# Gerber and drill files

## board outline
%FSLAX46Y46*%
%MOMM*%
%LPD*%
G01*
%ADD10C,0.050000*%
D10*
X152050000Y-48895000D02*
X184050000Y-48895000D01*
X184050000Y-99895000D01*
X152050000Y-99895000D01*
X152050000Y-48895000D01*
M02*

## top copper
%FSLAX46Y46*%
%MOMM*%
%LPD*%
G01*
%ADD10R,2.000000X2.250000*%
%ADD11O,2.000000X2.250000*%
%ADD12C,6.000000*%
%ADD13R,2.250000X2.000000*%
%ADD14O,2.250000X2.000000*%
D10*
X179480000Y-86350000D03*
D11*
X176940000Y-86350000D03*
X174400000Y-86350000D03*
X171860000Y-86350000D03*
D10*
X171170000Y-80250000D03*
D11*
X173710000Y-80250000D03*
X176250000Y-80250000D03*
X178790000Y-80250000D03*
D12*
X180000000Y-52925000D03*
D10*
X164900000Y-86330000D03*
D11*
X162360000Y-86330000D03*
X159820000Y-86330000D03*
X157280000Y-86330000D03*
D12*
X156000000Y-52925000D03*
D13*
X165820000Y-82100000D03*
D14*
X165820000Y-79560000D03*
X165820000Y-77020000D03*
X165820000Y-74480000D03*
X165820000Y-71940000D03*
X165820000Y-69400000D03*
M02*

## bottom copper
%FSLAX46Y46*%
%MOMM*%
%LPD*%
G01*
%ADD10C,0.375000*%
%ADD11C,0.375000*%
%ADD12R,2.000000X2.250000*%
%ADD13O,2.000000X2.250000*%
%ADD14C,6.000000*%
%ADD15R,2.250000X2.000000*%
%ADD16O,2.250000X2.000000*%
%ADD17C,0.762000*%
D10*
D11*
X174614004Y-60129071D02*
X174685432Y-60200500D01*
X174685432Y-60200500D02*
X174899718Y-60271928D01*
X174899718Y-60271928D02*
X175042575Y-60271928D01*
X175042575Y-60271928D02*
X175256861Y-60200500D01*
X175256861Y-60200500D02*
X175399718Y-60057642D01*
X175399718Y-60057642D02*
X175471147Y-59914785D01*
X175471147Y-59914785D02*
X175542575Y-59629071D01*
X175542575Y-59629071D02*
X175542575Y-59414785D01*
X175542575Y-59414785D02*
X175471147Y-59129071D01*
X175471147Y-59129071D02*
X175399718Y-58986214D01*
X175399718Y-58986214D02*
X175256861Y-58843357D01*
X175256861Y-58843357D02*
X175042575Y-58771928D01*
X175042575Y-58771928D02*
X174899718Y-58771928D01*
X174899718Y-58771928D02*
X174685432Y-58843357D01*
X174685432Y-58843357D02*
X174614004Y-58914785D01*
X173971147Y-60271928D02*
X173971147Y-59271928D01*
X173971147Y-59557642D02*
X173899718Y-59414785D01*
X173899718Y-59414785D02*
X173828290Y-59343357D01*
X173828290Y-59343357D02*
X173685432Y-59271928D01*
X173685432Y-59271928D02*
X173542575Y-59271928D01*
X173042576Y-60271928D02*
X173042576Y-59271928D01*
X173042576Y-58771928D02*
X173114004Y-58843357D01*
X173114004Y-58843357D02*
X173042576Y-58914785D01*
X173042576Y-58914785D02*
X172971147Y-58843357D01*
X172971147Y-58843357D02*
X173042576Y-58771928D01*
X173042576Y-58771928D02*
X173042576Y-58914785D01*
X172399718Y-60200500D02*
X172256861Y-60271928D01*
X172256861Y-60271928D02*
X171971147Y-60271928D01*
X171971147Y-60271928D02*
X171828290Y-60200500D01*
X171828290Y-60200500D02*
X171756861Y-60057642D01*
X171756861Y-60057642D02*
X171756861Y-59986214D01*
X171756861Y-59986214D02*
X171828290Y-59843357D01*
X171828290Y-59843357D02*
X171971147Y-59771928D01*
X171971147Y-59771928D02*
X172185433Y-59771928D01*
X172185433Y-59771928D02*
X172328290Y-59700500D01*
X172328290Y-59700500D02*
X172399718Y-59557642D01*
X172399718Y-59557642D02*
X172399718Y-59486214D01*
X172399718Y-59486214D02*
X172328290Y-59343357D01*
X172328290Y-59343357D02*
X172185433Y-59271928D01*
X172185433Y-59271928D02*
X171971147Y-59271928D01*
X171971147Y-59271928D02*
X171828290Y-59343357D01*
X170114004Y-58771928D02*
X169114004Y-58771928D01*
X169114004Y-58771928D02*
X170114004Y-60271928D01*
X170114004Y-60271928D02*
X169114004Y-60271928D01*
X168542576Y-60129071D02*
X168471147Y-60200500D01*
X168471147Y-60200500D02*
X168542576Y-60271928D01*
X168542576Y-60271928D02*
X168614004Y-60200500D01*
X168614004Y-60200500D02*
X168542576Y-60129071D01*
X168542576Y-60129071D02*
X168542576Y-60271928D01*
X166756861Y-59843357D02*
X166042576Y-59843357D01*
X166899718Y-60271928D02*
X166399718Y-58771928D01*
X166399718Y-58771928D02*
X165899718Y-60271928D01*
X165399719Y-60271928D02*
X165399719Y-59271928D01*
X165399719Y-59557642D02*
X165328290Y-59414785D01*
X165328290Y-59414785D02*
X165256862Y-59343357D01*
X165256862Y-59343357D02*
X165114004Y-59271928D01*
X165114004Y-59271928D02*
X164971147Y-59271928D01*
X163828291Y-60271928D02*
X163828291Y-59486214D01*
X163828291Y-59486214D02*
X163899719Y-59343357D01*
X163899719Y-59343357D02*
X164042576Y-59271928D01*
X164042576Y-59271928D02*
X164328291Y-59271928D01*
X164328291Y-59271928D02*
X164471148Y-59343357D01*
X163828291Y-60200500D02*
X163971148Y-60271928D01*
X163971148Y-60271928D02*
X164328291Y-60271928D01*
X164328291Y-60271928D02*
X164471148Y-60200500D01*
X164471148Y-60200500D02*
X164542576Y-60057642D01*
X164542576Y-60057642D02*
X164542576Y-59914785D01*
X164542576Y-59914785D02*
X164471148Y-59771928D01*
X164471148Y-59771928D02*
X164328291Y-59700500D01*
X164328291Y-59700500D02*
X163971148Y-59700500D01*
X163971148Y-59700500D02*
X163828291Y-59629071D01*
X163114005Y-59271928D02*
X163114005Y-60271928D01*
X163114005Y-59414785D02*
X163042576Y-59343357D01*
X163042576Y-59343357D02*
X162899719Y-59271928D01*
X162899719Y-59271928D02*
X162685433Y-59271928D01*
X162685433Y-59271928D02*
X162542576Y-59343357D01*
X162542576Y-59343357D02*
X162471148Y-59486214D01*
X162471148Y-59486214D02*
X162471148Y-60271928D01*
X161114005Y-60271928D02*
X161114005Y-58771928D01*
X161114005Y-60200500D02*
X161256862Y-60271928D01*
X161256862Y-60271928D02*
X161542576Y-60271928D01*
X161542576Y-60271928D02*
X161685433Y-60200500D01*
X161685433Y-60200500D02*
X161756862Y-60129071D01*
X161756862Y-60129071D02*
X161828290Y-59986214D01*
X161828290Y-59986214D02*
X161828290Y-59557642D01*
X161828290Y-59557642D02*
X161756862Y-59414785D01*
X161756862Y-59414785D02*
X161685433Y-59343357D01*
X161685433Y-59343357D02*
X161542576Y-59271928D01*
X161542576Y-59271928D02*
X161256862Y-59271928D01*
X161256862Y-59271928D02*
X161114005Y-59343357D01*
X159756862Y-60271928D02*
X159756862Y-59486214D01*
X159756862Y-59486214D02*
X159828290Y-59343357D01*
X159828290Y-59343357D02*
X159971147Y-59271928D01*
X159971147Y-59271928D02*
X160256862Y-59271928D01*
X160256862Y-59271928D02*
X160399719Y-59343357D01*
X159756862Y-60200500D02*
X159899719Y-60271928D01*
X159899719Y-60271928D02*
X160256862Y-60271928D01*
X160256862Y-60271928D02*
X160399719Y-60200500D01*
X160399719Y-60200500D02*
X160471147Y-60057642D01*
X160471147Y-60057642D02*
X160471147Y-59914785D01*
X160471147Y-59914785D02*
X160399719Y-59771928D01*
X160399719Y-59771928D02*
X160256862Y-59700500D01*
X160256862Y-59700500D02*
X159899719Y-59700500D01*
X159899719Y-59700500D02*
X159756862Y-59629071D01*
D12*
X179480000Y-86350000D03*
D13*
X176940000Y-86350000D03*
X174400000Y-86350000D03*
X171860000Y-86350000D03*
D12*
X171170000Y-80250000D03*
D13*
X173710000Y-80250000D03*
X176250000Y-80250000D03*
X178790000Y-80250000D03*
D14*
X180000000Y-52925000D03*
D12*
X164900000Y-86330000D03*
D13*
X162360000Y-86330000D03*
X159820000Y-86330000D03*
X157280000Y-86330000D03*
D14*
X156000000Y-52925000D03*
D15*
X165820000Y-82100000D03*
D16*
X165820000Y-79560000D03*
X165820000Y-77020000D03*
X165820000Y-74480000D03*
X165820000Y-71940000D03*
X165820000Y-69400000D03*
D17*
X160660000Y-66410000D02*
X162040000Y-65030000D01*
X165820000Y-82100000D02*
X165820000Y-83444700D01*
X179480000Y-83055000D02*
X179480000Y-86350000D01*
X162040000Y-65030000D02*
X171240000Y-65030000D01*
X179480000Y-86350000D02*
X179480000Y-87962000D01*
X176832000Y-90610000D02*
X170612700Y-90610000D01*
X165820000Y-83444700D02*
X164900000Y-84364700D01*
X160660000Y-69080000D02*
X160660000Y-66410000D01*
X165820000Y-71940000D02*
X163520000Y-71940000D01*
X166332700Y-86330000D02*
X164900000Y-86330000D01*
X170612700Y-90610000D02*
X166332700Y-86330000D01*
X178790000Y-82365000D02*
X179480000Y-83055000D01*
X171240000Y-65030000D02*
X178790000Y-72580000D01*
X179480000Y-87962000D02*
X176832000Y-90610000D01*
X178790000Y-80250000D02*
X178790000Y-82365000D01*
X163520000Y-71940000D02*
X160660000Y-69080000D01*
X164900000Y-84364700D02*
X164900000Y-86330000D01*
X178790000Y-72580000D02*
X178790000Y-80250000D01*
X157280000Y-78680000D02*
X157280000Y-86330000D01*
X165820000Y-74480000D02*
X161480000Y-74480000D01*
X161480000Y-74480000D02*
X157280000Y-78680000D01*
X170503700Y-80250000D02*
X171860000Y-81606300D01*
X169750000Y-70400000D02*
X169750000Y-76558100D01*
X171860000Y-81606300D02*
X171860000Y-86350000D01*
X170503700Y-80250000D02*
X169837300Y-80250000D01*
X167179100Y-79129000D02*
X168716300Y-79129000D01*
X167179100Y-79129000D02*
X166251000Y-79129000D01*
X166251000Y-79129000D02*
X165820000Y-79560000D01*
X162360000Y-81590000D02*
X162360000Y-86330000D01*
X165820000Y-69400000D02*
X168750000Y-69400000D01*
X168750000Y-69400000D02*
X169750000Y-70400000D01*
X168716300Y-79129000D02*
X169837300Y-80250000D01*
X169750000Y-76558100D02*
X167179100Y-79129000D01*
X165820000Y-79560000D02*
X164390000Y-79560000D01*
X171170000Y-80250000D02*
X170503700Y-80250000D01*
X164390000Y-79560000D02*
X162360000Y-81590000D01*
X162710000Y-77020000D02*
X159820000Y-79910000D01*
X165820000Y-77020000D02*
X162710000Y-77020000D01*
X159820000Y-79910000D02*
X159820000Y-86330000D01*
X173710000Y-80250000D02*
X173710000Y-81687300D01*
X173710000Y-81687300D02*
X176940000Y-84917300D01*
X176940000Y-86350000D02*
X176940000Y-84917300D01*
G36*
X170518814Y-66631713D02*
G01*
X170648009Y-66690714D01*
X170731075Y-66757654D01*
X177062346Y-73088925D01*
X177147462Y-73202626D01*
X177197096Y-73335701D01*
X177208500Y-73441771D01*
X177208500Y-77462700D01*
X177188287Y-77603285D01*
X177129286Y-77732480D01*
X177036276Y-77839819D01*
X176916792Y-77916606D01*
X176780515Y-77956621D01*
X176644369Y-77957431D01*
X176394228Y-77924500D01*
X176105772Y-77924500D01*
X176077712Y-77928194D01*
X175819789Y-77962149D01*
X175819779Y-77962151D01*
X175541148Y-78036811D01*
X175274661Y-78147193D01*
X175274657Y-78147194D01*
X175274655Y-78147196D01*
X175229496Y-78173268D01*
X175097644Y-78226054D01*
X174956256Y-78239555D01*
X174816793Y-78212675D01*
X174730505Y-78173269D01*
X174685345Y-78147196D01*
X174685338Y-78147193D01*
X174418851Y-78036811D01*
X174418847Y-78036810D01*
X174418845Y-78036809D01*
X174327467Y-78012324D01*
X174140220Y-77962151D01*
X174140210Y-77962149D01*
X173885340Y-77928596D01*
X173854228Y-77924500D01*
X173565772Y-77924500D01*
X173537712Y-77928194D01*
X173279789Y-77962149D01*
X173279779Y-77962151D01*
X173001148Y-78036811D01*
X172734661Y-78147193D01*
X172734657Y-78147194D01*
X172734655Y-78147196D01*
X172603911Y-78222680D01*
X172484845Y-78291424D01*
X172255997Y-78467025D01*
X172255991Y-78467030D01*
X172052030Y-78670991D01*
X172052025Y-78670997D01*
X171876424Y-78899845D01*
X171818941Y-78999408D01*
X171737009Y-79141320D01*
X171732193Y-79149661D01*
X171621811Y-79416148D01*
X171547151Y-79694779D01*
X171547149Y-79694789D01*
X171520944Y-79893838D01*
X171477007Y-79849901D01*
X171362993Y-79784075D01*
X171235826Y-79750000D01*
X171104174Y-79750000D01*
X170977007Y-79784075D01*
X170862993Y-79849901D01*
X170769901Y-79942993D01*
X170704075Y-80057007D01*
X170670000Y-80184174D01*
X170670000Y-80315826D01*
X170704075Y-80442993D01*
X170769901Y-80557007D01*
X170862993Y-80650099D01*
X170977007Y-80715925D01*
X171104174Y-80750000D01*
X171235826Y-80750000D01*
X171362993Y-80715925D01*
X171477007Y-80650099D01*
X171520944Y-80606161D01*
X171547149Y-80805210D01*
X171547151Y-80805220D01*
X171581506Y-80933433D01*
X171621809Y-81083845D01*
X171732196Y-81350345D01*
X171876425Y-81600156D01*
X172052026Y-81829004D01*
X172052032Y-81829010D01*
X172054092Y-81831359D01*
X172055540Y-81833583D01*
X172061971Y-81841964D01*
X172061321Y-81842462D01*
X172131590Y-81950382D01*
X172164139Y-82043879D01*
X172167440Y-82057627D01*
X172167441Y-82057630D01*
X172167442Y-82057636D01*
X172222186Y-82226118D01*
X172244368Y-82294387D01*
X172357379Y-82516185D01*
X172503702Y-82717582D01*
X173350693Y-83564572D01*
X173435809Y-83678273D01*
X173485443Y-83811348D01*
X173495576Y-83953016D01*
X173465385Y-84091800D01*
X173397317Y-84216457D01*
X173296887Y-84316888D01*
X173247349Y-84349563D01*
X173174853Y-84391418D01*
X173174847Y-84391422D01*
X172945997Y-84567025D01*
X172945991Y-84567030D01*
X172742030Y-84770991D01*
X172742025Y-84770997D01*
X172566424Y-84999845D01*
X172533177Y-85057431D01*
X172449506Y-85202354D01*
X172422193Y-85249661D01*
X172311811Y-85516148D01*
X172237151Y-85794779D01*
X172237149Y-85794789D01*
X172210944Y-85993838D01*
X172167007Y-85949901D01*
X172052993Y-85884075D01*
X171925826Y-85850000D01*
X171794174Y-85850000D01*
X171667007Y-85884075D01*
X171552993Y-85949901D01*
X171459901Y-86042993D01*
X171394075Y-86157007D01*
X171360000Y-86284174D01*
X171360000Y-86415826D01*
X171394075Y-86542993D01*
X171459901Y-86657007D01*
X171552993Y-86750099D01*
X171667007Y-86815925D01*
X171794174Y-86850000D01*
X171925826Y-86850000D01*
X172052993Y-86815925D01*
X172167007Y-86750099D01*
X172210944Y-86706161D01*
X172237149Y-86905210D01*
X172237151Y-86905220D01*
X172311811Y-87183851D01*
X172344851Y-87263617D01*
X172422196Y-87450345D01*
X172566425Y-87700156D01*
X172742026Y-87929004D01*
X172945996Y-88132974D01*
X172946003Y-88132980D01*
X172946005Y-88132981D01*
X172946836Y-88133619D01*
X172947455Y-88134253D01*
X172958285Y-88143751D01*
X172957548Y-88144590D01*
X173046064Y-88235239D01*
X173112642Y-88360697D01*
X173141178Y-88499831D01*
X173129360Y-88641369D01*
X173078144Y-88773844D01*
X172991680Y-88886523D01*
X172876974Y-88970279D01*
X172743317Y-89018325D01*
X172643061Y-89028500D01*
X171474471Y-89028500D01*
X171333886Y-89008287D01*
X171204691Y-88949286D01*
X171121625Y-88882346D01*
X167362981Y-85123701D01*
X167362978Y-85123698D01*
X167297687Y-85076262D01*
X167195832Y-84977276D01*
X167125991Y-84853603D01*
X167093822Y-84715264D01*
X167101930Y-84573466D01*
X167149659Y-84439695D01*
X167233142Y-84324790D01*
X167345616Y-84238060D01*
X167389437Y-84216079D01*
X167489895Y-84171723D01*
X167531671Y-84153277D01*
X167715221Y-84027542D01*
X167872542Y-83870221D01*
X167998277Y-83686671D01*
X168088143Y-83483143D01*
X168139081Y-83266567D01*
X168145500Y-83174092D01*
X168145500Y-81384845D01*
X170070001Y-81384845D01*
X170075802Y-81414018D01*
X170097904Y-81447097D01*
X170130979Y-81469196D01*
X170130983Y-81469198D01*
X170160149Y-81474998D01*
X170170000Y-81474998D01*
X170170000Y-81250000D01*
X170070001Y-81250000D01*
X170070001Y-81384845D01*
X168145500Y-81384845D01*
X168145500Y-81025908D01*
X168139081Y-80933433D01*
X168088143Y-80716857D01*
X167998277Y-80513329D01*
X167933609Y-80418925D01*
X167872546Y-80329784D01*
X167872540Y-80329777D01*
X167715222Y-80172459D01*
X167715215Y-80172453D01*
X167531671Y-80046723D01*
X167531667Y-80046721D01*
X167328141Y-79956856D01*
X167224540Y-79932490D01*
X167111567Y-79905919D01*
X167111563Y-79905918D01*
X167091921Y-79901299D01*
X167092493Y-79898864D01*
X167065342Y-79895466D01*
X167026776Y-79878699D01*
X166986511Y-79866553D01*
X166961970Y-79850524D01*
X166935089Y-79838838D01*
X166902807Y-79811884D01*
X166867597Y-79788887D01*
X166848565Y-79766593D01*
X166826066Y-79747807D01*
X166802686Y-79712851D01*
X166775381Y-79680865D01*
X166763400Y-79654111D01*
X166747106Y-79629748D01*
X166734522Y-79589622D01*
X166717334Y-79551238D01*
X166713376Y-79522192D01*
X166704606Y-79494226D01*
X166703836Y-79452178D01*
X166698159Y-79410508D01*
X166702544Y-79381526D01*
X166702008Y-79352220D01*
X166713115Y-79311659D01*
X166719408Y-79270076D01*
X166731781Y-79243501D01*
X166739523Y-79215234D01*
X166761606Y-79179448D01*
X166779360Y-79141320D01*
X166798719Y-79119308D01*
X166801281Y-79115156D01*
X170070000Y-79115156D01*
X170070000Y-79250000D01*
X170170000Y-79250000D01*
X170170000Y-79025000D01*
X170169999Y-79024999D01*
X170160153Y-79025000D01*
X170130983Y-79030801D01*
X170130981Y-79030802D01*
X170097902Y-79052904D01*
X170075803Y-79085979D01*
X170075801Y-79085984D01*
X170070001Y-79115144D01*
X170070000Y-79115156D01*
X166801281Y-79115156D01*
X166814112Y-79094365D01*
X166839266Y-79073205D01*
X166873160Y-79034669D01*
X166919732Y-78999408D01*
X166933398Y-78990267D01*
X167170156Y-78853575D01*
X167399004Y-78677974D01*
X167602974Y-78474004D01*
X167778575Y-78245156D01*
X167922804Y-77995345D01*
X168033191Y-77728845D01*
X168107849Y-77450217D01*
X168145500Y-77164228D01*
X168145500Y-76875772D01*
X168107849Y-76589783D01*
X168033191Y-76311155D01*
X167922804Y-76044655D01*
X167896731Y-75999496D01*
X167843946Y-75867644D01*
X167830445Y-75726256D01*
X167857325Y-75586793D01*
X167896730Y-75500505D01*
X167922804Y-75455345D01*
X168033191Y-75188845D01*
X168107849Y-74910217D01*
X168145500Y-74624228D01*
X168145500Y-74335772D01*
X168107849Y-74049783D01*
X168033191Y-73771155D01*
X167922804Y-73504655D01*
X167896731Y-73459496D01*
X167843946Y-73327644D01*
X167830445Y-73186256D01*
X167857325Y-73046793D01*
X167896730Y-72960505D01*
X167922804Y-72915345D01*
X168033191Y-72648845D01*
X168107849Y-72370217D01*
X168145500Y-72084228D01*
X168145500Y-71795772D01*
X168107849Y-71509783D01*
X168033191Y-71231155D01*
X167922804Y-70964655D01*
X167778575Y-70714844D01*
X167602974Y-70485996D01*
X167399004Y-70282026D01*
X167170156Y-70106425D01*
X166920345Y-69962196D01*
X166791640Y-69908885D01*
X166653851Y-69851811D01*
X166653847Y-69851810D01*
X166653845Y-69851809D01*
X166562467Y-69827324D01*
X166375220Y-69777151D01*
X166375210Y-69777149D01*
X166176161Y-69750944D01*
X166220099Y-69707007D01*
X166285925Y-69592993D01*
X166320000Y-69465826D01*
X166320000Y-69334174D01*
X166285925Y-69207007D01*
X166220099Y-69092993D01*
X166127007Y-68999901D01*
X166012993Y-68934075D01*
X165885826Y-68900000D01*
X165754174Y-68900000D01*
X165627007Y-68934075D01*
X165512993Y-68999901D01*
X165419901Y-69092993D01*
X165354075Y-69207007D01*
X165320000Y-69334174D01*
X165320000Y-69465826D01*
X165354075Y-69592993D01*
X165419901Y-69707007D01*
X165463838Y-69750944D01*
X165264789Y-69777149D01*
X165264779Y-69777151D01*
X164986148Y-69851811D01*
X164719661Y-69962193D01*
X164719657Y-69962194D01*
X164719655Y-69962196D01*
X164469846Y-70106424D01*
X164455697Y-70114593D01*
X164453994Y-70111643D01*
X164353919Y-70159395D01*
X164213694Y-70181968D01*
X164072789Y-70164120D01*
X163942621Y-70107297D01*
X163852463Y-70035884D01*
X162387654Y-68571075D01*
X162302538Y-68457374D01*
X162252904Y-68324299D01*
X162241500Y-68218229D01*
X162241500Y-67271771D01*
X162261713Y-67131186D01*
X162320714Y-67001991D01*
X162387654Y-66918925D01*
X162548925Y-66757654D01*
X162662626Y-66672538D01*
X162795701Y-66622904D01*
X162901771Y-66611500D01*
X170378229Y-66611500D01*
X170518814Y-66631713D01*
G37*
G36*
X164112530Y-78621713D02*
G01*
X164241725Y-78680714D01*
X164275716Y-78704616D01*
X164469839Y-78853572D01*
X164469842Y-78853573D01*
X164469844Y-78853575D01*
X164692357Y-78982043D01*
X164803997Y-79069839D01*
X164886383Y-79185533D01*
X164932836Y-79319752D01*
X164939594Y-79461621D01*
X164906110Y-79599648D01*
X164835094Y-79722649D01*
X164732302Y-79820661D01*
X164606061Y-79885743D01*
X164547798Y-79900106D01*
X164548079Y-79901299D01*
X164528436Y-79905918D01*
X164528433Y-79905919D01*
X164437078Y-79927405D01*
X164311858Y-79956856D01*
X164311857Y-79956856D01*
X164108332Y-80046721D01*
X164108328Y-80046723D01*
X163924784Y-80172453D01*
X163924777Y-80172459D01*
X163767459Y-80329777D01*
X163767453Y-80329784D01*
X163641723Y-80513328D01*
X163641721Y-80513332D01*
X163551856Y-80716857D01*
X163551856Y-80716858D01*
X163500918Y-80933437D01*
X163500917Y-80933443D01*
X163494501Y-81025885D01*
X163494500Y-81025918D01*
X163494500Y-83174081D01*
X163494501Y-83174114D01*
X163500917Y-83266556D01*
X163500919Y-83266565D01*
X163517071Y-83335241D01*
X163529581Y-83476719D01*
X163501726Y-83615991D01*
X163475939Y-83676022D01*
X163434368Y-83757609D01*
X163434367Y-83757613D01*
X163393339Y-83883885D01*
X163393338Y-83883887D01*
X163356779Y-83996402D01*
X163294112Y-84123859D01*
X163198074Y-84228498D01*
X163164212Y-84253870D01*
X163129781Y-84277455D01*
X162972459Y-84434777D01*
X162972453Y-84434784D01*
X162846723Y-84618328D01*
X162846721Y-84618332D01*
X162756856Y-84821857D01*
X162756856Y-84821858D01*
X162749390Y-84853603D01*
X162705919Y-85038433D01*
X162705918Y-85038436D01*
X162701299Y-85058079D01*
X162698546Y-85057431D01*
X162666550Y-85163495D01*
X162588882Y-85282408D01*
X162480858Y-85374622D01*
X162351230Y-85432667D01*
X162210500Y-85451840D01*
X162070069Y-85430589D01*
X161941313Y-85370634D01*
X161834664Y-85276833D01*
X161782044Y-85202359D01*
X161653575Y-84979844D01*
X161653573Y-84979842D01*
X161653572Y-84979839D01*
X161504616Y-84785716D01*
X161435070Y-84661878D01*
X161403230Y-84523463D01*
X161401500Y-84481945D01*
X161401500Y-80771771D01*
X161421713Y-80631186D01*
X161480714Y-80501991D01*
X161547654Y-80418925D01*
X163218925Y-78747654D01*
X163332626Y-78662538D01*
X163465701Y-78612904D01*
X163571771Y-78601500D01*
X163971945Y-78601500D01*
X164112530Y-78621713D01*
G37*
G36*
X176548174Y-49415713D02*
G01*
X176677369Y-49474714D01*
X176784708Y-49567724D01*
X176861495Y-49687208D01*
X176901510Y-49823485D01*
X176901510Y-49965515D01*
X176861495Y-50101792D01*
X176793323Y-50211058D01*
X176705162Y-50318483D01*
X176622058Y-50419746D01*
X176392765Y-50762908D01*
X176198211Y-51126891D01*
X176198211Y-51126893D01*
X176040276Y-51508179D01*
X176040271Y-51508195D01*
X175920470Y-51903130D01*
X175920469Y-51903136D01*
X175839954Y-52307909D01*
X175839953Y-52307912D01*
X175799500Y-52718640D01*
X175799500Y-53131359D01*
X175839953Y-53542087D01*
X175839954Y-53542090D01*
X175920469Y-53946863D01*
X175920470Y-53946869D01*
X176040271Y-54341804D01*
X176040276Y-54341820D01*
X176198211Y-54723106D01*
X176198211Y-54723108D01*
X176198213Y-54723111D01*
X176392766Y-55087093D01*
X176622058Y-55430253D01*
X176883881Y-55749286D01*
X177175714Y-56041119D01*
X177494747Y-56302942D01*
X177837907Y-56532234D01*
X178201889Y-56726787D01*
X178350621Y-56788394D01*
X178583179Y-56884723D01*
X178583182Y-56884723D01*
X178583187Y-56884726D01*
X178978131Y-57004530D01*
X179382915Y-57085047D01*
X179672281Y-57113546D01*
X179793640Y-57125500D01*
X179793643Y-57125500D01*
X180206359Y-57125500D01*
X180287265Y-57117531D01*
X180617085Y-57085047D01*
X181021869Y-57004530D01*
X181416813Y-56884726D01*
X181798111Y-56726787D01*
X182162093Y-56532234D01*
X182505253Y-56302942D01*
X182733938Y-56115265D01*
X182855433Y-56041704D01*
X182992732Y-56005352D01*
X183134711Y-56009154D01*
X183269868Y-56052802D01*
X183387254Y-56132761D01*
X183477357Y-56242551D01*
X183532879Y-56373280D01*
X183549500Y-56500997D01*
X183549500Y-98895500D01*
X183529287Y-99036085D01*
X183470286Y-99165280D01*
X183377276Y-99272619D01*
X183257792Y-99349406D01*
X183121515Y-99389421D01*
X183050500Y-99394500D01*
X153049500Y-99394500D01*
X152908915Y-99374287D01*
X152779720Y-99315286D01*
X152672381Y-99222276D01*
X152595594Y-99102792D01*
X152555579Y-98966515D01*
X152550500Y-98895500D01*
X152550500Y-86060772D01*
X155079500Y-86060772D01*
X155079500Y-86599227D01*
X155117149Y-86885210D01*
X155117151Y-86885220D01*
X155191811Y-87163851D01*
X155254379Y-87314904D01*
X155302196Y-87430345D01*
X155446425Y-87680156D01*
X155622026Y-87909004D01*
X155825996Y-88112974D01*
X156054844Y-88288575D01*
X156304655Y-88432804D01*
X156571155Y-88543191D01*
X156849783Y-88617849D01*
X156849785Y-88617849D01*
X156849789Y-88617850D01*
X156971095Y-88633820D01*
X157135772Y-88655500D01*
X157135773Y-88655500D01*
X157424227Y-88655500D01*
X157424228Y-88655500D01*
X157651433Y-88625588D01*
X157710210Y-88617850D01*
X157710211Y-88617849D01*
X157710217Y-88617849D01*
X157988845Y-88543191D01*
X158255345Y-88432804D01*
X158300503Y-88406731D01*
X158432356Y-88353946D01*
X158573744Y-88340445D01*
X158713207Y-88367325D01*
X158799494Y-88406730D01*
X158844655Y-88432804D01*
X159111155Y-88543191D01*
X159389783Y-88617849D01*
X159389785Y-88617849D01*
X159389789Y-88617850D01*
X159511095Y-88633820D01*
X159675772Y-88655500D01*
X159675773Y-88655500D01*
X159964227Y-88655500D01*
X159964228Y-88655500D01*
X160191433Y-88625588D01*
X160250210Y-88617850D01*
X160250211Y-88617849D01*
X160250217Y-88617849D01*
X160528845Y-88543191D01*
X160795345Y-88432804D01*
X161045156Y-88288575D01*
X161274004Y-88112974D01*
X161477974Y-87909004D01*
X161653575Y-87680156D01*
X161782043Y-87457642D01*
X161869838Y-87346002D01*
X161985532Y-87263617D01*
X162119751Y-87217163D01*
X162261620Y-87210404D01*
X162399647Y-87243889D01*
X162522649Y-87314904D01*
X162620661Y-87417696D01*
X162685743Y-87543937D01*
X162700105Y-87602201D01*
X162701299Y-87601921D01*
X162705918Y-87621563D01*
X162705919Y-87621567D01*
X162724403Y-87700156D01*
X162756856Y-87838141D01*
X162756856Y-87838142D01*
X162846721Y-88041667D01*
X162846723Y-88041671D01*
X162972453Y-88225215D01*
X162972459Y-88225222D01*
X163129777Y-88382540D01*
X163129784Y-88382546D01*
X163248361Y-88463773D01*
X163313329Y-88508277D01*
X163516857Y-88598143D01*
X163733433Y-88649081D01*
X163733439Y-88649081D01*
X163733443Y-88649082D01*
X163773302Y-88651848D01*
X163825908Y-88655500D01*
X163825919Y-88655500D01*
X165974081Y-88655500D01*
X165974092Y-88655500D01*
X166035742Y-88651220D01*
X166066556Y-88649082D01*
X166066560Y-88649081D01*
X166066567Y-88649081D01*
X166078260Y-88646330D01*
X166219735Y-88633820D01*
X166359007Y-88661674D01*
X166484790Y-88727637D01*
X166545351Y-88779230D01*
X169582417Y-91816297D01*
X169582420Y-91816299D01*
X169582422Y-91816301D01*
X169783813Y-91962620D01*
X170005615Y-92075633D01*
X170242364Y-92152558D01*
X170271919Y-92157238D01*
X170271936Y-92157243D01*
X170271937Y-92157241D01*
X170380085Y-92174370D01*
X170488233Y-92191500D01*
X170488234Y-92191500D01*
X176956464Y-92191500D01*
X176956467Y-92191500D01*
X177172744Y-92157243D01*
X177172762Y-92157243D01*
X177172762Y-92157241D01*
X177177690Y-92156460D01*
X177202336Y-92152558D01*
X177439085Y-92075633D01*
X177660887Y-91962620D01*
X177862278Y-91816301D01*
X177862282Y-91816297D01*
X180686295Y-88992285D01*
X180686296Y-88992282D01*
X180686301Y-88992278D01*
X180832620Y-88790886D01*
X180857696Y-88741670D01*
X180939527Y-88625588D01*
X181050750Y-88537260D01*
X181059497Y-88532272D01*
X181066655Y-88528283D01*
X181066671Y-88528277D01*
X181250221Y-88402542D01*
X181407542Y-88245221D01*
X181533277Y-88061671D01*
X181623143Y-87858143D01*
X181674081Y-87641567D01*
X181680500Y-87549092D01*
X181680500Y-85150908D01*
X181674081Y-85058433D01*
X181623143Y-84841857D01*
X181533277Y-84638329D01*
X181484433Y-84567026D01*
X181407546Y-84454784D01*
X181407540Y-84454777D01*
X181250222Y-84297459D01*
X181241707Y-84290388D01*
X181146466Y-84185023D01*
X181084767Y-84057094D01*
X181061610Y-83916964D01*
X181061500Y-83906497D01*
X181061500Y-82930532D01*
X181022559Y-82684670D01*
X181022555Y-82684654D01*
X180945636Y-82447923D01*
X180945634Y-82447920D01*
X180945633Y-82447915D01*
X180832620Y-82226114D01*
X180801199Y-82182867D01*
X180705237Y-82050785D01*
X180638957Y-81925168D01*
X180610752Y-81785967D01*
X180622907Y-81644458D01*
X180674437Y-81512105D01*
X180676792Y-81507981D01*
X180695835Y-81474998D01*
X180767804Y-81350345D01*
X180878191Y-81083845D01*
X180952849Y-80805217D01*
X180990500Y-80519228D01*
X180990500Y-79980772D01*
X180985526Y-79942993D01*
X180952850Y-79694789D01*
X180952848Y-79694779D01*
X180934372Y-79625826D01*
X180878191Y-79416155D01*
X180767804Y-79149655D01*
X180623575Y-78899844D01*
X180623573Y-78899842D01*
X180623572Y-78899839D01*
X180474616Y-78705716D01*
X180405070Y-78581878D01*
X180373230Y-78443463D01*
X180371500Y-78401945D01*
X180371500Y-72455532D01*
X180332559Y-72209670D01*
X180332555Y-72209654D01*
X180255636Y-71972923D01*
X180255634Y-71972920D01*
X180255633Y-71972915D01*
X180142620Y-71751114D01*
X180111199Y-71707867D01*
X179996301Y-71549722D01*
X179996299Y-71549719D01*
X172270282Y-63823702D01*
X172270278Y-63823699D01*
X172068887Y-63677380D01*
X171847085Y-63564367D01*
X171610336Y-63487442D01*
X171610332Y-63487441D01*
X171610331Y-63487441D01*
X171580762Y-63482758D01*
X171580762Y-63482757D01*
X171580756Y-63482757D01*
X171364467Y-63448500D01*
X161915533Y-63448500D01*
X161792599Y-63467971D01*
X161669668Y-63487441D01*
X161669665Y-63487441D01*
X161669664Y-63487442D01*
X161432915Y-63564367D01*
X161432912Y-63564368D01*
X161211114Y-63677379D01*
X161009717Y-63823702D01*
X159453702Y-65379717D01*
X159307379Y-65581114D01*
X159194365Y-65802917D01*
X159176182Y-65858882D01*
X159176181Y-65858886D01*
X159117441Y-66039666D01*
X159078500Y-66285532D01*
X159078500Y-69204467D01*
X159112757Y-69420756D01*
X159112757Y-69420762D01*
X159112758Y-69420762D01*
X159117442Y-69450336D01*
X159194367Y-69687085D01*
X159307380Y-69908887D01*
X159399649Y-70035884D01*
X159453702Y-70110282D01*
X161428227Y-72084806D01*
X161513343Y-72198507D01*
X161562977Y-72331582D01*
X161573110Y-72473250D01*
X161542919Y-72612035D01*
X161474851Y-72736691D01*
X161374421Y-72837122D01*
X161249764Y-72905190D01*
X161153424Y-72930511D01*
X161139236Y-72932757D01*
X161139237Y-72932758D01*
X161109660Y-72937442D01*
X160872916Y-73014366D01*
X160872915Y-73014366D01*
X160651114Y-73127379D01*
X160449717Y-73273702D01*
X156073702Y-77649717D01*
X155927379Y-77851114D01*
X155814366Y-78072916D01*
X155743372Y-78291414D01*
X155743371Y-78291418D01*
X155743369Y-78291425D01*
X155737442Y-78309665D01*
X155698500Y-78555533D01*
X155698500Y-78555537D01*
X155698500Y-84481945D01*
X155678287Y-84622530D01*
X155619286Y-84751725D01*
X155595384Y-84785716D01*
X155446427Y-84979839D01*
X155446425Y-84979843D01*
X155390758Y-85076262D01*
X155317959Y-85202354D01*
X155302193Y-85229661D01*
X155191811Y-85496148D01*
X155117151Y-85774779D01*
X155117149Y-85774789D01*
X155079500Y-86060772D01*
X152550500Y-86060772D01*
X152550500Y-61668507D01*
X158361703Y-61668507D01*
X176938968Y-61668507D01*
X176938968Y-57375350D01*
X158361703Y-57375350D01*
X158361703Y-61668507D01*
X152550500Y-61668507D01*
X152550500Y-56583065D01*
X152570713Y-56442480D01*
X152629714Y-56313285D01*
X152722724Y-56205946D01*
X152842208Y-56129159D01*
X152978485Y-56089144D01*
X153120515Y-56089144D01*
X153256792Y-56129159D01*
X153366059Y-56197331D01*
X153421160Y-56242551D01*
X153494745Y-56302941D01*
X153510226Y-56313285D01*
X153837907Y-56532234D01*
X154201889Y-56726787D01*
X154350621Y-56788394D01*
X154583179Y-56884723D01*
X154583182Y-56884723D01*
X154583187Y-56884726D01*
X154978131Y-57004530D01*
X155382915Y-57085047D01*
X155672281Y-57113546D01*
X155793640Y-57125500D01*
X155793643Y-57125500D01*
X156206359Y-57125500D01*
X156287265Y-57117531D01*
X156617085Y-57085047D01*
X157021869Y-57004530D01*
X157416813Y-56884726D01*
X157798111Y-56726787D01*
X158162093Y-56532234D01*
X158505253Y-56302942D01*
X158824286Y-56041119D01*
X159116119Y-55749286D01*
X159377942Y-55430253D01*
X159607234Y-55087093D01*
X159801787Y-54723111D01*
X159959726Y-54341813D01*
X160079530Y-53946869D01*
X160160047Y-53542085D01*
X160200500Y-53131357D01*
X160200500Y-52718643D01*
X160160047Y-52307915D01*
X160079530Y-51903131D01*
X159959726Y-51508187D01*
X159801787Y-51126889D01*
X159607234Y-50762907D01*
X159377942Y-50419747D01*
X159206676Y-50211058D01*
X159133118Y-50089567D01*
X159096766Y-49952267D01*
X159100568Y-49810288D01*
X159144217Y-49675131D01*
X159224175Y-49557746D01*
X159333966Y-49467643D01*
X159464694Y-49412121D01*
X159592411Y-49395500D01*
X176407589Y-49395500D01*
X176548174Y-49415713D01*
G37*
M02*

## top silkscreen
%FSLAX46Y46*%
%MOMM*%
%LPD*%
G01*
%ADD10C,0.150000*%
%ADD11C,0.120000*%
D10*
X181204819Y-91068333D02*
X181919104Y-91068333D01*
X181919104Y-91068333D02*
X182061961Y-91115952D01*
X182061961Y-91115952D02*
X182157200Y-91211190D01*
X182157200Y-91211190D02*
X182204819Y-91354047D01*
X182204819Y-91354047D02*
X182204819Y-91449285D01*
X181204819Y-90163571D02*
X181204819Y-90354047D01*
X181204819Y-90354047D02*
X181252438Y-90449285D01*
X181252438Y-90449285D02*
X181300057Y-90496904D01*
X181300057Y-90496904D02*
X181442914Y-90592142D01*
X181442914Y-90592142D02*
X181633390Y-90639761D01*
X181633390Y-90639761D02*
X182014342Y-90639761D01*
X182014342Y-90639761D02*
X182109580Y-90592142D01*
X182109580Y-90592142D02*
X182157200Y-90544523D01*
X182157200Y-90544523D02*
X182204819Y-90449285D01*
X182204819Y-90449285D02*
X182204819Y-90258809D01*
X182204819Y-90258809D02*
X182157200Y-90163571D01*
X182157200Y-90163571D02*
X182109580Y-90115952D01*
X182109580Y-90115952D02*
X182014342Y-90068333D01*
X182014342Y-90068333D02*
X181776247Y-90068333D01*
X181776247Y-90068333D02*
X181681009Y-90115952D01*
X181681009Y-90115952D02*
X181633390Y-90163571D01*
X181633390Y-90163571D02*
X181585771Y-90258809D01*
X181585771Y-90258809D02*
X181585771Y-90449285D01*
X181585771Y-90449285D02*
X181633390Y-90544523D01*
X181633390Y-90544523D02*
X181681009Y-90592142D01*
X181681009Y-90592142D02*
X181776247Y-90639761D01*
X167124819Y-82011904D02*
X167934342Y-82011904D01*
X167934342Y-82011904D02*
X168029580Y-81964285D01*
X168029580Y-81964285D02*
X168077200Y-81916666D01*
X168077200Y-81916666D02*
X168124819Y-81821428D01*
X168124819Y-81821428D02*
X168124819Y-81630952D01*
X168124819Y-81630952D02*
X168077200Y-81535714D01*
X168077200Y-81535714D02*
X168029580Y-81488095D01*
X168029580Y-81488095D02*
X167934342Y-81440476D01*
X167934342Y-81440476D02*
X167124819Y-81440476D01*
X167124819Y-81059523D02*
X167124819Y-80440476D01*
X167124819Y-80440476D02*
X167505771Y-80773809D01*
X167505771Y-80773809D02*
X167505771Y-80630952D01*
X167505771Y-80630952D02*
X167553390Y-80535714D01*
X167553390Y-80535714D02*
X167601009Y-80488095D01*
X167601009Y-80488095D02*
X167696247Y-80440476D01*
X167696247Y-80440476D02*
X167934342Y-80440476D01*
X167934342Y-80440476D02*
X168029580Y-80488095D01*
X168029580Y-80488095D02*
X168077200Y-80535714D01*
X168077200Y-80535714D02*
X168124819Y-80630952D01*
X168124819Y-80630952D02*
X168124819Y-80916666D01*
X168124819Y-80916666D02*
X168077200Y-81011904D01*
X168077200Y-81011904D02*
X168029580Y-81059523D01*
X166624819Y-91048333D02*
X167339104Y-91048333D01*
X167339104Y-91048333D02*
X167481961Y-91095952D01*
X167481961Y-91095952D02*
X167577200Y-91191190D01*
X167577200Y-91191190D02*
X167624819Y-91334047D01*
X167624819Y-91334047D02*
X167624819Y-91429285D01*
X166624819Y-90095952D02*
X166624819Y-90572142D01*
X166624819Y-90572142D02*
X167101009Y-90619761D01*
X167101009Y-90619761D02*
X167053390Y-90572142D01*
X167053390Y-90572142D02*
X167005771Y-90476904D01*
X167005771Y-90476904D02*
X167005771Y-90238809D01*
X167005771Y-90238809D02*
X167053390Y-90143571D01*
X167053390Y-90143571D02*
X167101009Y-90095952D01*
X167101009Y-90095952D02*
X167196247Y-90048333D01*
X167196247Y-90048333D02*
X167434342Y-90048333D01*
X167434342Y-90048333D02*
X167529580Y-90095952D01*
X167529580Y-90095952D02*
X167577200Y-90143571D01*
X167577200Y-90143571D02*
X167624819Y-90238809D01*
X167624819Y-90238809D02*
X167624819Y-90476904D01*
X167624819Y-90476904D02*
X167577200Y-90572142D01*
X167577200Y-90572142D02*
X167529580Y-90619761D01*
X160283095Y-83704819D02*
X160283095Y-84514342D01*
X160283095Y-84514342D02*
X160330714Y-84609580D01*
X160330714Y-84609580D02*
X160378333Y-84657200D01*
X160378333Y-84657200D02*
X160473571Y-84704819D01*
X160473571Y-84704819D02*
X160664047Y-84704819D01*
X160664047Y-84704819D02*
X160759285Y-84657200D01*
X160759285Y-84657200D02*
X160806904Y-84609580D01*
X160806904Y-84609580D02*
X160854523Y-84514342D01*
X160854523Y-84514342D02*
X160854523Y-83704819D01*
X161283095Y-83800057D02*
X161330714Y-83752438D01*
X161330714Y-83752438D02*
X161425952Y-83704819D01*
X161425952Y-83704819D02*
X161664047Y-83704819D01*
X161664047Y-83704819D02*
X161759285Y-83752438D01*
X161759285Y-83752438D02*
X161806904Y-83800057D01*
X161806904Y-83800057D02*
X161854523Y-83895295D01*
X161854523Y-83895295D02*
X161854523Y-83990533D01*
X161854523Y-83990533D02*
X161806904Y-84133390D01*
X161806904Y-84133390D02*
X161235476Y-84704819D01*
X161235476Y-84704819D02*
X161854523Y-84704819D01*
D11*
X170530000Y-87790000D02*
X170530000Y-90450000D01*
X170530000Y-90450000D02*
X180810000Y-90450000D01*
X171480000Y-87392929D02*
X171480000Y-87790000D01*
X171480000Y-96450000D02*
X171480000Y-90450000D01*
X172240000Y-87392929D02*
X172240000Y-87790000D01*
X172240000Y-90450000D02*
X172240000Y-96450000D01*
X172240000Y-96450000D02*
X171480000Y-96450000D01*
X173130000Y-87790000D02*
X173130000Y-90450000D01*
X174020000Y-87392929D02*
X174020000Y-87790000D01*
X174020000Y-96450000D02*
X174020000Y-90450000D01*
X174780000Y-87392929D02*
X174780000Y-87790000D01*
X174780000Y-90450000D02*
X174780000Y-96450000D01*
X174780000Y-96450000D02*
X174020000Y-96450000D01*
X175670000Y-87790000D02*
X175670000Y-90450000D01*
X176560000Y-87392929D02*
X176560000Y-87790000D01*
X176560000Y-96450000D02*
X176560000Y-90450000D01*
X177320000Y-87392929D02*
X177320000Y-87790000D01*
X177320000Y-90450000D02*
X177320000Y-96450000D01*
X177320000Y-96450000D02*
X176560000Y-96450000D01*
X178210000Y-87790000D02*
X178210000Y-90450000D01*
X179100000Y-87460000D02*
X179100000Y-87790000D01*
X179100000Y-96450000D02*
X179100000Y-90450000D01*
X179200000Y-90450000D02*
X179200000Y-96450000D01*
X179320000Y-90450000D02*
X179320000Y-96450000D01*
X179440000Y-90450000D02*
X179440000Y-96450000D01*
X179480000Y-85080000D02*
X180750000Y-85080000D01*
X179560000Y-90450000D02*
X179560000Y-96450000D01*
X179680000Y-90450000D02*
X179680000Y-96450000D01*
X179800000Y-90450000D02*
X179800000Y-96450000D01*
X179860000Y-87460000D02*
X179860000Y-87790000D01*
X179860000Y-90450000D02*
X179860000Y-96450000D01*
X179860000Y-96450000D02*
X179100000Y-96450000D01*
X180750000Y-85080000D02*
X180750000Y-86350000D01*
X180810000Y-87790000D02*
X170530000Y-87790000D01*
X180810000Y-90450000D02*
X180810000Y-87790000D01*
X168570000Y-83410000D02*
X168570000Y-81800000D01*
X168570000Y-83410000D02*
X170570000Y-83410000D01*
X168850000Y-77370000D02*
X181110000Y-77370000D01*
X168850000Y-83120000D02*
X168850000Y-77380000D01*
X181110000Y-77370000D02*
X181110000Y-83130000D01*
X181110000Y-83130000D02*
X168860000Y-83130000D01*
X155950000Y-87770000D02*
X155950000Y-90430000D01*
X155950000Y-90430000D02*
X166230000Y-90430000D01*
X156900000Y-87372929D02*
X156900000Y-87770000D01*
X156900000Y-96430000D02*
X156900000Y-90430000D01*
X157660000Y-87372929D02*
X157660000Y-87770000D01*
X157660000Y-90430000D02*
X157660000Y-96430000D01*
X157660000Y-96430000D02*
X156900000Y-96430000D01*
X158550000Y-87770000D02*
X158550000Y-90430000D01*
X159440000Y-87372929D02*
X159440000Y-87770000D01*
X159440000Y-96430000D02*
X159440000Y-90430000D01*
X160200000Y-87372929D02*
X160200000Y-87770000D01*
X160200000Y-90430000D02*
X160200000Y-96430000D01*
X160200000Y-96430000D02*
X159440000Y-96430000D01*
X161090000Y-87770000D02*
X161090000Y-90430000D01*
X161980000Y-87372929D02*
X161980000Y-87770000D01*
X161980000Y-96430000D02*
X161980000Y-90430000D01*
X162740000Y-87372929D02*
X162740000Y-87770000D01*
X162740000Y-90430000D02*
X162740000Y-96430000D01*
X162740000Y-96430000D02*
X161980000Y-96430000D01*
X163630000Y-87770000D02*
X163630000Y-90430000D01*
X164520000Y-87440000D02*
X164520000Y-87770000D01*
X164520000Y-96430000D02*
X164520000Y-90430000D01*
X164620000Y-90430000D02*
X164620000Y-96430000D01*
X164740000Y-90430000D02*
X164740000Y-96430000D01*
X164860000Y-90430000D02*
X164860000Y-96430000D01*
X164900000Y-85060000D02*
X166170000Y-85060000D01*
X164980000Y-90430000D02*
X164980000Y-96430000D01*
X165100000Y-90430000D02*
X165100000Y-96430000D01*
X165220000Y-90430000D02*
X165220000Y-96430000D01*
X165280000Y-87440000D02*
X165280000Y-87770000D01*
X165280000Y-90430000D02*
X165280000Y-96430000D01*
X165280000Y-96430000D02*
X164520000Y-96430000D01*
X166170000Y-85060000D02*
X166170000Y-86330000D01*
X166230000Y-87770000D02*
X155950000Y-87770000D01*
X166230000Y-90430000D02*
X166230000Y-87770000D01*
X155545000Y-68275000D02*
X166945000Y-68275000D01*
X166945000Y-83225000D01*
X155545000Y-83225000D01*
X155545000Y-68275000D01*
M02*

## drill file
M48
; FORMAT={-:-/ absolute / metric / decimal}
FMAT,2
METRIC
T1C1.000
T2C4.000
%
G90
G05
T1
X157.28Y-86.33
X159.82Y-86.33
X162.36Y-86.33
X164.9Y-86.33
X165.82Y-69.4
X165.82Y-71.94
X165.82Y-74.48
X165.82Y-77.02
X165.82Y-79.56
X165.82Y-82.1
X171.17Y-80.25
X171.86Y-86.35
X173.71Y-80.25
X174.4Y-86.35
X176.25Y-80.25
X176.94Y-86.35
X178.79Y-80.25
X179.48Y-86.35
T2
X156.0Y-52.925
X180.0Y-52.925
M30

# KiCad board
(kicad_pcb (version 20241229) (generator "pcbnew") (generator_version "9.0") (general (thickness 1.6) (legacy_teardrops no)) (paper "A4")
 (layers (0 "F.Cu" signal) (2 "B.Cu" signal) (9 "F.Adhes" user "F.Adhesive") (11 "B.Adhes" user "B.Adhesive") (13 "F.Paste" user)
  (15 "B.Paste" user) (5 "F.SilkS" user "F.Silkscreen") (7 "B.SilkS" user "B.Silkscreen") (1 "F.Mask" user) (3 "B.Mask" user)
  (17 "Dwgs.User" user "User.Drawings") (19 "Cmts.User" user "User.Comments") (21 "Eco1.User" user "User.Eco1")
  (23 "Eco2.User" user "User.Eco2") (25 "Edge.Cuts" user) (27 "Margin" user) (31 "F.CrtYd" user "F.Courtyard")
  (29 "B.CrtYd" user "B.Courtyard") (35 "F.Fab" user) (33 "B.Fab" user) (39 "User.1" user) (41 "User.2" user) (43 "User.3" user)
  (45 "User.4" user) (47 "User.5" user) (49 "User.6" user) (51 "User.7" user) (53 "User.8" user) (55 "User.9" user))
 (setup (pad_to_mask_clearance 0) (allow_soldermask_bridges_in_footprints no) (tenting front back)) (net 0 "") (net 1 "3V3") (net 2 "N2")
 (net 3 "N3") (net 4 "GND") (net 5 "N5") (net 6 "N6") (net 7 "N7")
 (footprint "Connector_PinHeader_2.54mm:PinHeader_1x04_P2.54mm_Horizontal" (layer "F.Cu") (at 179.48 86.35 -90)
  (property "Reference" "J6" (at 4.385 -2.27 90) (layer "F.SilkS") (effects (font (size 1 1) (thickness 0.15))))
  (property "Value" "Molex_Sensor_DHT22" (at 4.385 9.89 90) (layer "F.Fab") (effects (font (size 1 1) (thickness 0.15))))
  (fp_line (start 1.44 8.95) (end 4.1 8.95) (stroke (width 0.12) (type solid)) (layer "F.SilkS"))
  (fp_line (start 4.1 8.95) (end 4.1 -1.33) (stroke (width 0.12) (type solid)) (layer "F.SilkS"))
  (fp_line (start 1.042929 8) (end 1.44 8) (stroke (width 0.12) (type solid)) (layer "F.SilkS"))
  (fp_line (start 10.1 8) (end 4.1 8) (stroke (width 0.12) (type solid)) (layer "F.SilkS"))
  (fp_line (start 1.042929 7.24) (end 1.44 7.24) (stroke (width 0.12) (type solid)) (layer "F.SilkS"))
  (fp_line (start 4.1 7.24) (end 10.1 7.24) (stroke (width 0.12) (type solid)) (layer "F.SilkS"))
  (fp_line (start 10.1 7.24) (end 10.1 8) (stroke (width 0.12) (type solid)) (layer "F.SilkS"))
  (fp_line (start 1.44 6.35) (end 4.1 6.35) (stroke (width 0.12) (type solid)) (layer "F.SilkS"))
  (fp_line (start 1.042929 5.46) (end 1.44 5.46) (stroke (width 0.12) (type solid)) (layer "F.SilkS"))
  (fp_line (start 10.1 5.46) (end 4.1 5.46) (stroke (width 0.12) (type solid)) (layer "F.SilkS"))
  (fp_line (start 1.042929 4.7) (end 1.44 4.7) (stroke (width 0.12) (type solid)) (layer "F.SilkS"))
  (fp_line (start 4.1 4.7) (end 10.1 4.7) (stroke (width 0.12) (type solid)) (layer "F.SilkS"))
  (fp_line (start 10.1 4.7) (end 10.1 5.46) (stroke (width 0.12) (type solid)) (layer "F.SilkS"))
  (fp_line (start 1.44 3.81) (end 4.1 3.81) (stroke (width 0.12) (type solid)) (layer "F.SilkS"))
  (fp_line (start 1.042929 2.92) (end 1.44 2.92) (stroke (width 0.12) (type solid)) (layer "F.SilkS"))
  (fp_line (start 10.1 2.92) (end 4.1 2.92) (stroke (width 0.12) (type solid)) (layer "F.SilkS"))
  (fp_line (start 1.042929 2.16) (end 1.44 2.16) (stroke (width 0.12) (type solid)) (layer "F.SilkS"))
  (fp_line (start 4.1 2.16) (end 10.1 2.16) (stroke (width 0.12) (type solid)) (layer "F.SilkS"))
  (fp_line (start 10.1 2.16) (end 10.1 2.92) (stroke (width 0.12) (type solid)) (layer "F.SilkS"))
  (fp_line (start 1.44 1.27) (end 4.1 1.27) (stroke (width 0.12) (type solid)) (layer "F.SilkS"))
  (fp_line (start 1.11 0.38) (end 1.44 0.38) (stroke (width 0.12) (type solid)) (layer "F.SilkS"))
  (fp_line (start 10.1 0.38) (end 4.1 0.38) (stroke (width 0.12) (type solid)) (layer "F.SilkS"))
  (fp_line (start 4.1 0.28) (end 10.1 0.28) (stroke (width 0.12) (type solid)) (layer "F.SilkS"))
  (fp_line (start 4.1 0.16) (end 10.1 0.16) (stroke (width 0.12) (type solid)) (layer "F.SilkS"))
  (fp_line (start 4.1 0.04) (end 10.1 0.04) (stroke (width 0.12) (type solid)) (layer "F.SilkS"))
  (fp_line (start -1.27 0) (end -1.27 -1.27) (stroke (width 0.12) (type solid)) (layer "F.SilkS"))
  (fp_line (start 4.1 -0.08) (end 10.1 -0.08) (stroke (width 0.12) (type solid)) (layer "F.SilkS"))
  (fp_line (start 4.1 -0.2) (end 10.1 -0.2) (stroke (width 0.12) (type solid)) (layer "F.SilkS"))
  (fp_line (start 4.1 -0.32) (end 10.1 -0.32) (stroke (width 0.12) (type solid)) (layer "F.SilkS"))
  (fp_line (start 1.11 -0.38) (end 1.44 -0.38) (stroke (width 0.12) (type solid)) (layer "F.SilkS"))
  (fp_line (start 4.1 -0.38) (end 10.1 -0.38) (stroke (width 0.12) (type solid)) (layer "F.SilkS"))
  (fp_line (start 10.1 -0.38) (end 10.1 0.38) (stroke (width 0.12) (type solid)) (layer "F.SilkS"))
  (fp_line (start -1.27 -1.27) (end 0 -1.27) (stroke (width 0.12) (type solid)) (layer "F.SilkS"))
  (fp_line (start 1.44 -1.33) (end 1.44 8.95) (stroke (width 0.12) (type solid)) (layer "F.SilkS"))
  (fp_line (start 4.1 -1.33) (end 1.44 -1.33) (stroke (width 0.12) (type solid)) (layer "F.SilkS"))
  (pad "1" thru_hole rect (at 0 0 270) (size 2.25 2) (drill 1) (layers "*.Cu" "*.Mask") (remove_unused_layers no) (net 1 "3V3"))
  (pad "2" thru_hole oval (at 0 2.54 270) (size 2.25 2) (drill 1) (layers "*.Cu" "*.Mask") (remove_unused_layers no) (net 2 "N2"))
  (pad "3" thru_hole oval (at 0 5.08 270) (size 2.25 2) (drill 1) (layers "*.Cu" "*.Mask") (remove_unused_layers no) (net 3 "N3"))
  (pad "4" thru_hole oval (at 0 7.62 270) (size 2.25 2) (drill 1) (layers "*.Cu" "*.Mask") (remove_unused_layers no) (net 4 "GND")))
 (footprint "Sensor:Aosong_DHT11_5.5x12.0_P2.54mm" (layer "F.Cu") (at 171.17 80.25 90)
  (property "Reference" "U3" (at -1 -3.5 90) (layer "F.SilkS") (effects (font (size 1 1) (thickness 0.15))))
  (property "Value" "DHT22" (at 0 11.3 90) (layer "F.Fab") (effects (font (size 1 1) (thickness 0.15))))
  (fp_line (start -3.16 -2.6) (end -1.55 -2.6) (stroke (width 0.12) (type solid)) (layer "F.SilkS"))
  (fp_line (start -3.16 -2.6) (end -3.16 -0.6) (stroke (width 0.12) (type solid)) (layer "F.SilkS"))
  (fp_line (start 2.88 -2.32) (end 2.88 9.94) (stroke (width 0.12) (type solid)) (layer "F.SilkS"))
  (fp_line (start -2.87 -2.32) (end 2.87 -2.32) (stroke (width 0.12) (type solid)) (layer "F.SilkS"))
  (fp_line (start 2.88 9.94) (end -2.88 9.94) (stroke (width 0.12) (type solid)) (layer "F.SilkS"))
  (fp_line (start -2.88 9.94) (end -2.88 -2.31) (stroke (width 0.12) (type solid)) (layer "F.SilkS"))
  (pad "1" thru_hole rect (at 0 0 90) (size 2.25 2) (drill 1) (layers "*.Cu" "*.Mask") (remove_unused_layers no) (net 4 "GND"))
  (pad "2" thru_hole oval (at 0 2.54 90) (size 2.25 2) (drill 1) (layers "*.Cu" "*.Mask") (remove_unused_layers no) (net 2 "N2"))
  (pad "3" thru_hole oval (at 0 5.08 90) (size 2.25 2) (drill 1) (layers "*.Cu" "*.Mask") (remove_unused_layers no) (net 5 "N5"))
  (pad "4" thru_hole oval (at 0 7.62 90) (size 2.25 2) (drill 1) (layers "*.Cu" "*.Mask") (remove_unused_layers no) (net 1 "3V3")))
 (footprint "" (layer "F.Cu") (at 180 52.925)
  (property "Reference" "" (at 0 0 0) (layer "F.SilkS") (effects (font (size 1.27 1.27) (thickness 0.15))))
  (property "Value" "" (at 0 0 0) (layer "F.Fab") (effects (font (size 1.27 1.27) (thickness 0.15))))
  (pad "" thru_hole circle (at 0 0 180) (size 6 6) (drill 4) (layers "*.Cu" "*.Mask") (remove_unused_layers no)))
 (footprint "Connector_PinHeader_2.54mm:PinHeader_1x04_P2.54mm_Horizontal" (layer "F.Cu") (at 164.9 86.33 -90)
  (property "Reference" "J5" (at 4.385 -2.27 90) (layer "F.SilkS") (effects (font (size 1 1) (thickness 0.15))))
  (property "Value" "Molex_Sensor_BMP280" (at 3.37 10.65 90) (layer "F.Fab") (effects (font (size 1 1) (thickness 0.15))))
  (fp_line (start 1.44 8.95) (end 4.1 8.95) (stroke (width 0.12) (type solid)) (layer "F.SilkS"))
  (fp_line (start 4.1 8.95) (end 4.1 -1.33) (stroke (width 0.12) (type solid)) (layer "F.SilkS"))
  (fp_line (start 1.042929 8) (end 1.44 8) (stroke (width 0.12) (type solid)) (layer "F.SilkS"))
  (fp_line (start 10.1 8) (end 4.1 8) (stroke (width 0.12) (type solid)) (layer "F.SilkS"))
  (fp_line (start 1.042929 7.24) (end 1.44 7.24) (stroke (width 0.12) (type solid)) (layer "F.SilkS"))
  (fp_line (start 4.1 7.24) (end 10.1 7.24) (stroke (width 0.12) (type solid)) (layer "F.SilkS"))
  (fp_line (start 10.1 7.24) (end 10.1 8) (stroke (width 0.12) (type solid)) (layer "F.SilkS"))
  (fp_line (start 1.44 6.35) (end 4.1 6.35) (stroke (width 0.12) (type solid)) (layer "F.SilkS"))
  (fp_line (start 1.042929 5.46) (end 1.44 5.46) (stroke (width 0.12) (type solid)) (layer "F.SilkS"))
  (fp_line (start 10.1 5.46) (end 4.1 5.46) (stroke (width 0.12) (type solid)) (layer "F.SilkS"))
  (fp_line (start 1.042929 4.7) (end 1.44 4.7) (stroke (width 0.12) (type solid)) (layer "F.SilkS"))
  (fp_line (start 4.1 4.7) (end 10.1 4.7) (stroke (width 0.12) (type solid)) (layer "F.SilkS"))
  (fp_line (start 10.1 4.7) (end 10.1 5.46) (stroke (width 0.12) (type solid)) (layer "F.SilkS"))
  (fp_line (start 1.44 3.81) (end 4.1 3.81) (stroke (width 0.12) (type solid)) (layer "F.SilkS"))
  (fp_line (start 1.042929 2.92) (end 1.44 2.92) (stroke (width 0.12) (type solid)) (layer "F.SilkS"))
  (fp_line (start 10.1 2.92) (end 4.1 2.92) (stroke (width 0.12) (type solid)) (layer "F.SilkS"))
  (fp_line (start 1.042929 2.16) (end 1.44 2.16) (stroke (width 0.12) (type solid)) (layer "F.SilkS"))
  (fp_line (start 4.1 2.16) (end 10.1 2.16) (stroke (width 0.12) (type solid)) (layer "F.SilkS"))
  (fp_line (start 10.1 2.16) (end 10.1 2.92) (stroke (width 0.12) (type solid)) (layer "F.SilkS"))
  (fp_line (start 1.44 1.27) (end 4.1 1.27) (stroke (width 0.12) (type solid)) (layer "F.SilkS"))
  (fp_line (start 1.11 0.38) (end 1.44 0.38) (stroke (width 0.12) (type solid)) (layer "F.SilkS"))
  (fp_line (start 10.1 0.38) (end 4.1 0.38) (stroke (width 0.12) (type solid)) (layer "F.SilkS"))
  (fp_line (start 4.1 0.28) (end 10.1 0.28) (stroke (width 0.12) (type solid)) (layer "F.SilkS"))
  (fp_line (start 4.1 0.16) (end 10.1 0.16) (stroke (width 0.12) (type solid)) (layer "F.SilkS"))
  (fp_line (start 4.1 0.04) (end 10.1 0.04) (stroke (width 0.12) (type solid)) (layer "F.SilkS"))
  (fp_line (start -1.27 0) (end -1.27 -1.27) (stroke (width 0.12) (type solid)) (layer "F.SilkS"))
  (fp_line (start 4.1 -0.08) (end 10.1 -0.08) (stroke (width 0.12) (type solid)) (layer "F.SilkS"))
  (fp_line (start 4.1 -0.2) (end 10.1 -0.2) (stroke (width 0.12) (type solid)) (layer "F.SilkS"))
  (fp_line (start 4.1 -0.32) (end 10.1 -0.32) (stroke (width 0.12) (type solid)) (layer "F.SilkS"))
  (fp_line (start 1.11 -0.38) (end 1.44 -0.38) (stroke (width 0.12) (type solid)) (layer "F.SilkS"))
  (fp_line (start 4.1 -0.38) (end 10.1 -0.38) (stroke (width 0.12) (type solid)) (layer "F.SilkS"))
  (fp_line (start 10.1 -0.38) (end 10.1 0.38) (stroke (width 0.12) (type solid)) (layer "F.SilkS"))
  (fp_line (start -1.27 -1.27) (end 0 -1.27) (stroke (width 0.12) (type solid)) (layer "F.SilkS"))
  (fp_line (start 1.44 -1.33) (end 1.44 8.95) (stroke (width 0.12) (type solid)) (layer "F.SilkS"))
  (fp_line (start 4.1 -1.33) (end 1.44 -1.33) (stroke (width 0.12) (type solid)) (layer "F.SilkS"))
  (pad "1" thru_hole rect (at 0 0 270) (size 2.25 2) (drill 1) (layers "*.Cu" "*.Mask") (remove_unused_layers no) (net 1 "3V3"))
  (pad "2" thru_hole oval (at 0 2.54 270) (size 2.25 2) (drill 1) (layers "*.Cu" "*.Mask") (remove_unused_layers no) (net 4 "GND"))
  (pad "3" thru_hole oval (at 0 5.08 270) (size 2.25 2) (drill 1) (layers "*.Cu" "*.Mask") (remove_unused_layers no) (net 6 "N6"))
  (pad "4" thru_hole oval (at 0 7.62 270) (size 2.25 2) (drill 1) (layers "*.Cu" "*.Mask") (remove_unused_layers no) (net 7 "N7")))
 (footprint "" (layer "F.Cu") (at 156 52.925)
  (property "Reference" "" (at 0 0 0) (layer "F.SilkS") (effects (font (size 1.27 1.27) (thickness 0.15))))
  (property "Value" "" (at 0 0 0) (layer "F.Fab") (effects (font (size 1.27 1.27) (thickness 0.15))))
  (pad "" thru_hole circle (at 0 0 180) (size 6 6) (drill 4) (layers "*.Cu" "*.Mask") (remove_unused_layers no)))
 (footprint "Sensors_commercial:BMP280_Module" (layer "F.Cu") (at 165.82 82.1 180)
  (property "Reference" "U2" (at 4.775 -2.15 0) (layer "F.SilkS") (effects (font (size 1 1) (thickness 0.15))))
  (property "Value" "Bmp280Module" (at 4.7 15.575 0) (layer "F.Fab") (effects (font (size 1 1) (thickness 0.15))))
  (fp_rect (start -1.125 -1.125) (end 10.275 13.825) (stroke (width 0.12) (type solid)) (fill no) (layer "F.SilkS"))
  (pad "1" thru_hole rect (at 0 0 180) (size 2.25 2) (drill 1) (layers "*.Cu" "*.Mask") (remove_unused_layers no) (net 1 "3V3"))
  (pad "2" thru_hole oval (at 0 2.54 180) (size 2.25 2) (drill 1) (layers "*.Cu" "*.Mask") (remove_unused_layers no) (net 4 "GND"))
  (pad "3" thru_hole oval (at 0 5.08 180) (size 2.25 2) (drill 1) (layers "*.Cu" "*.Mask") (remove_unused_layers no) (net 6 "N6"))
  (pad "4" thru_hole oval (at 0 7.62 180) (size 2.25 2) (drill 1) (layers "*.Cu" "*.Mask") (remove_unused_layers no) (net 7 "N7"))
  (pad "5" thru_hole oval (at 0 10.16 180) (size 2.25 2) (drill 1) (layers "*.Cu" "*.Mask") (remove_unused_layers no) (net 1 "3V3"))
  (pad "6" thru_hole oval (at 0 12.7 180) (size 2.25 2) (drill 1) (layers "*.Cu" "*.Mask") (remove_unused_layers no) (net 4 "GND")))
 (gr_rect (start 152.05 48.895) (end 184.05 99.895) (stroke (width 0.05) (type solid)) (fill no) (layer "Edge.Cuts"))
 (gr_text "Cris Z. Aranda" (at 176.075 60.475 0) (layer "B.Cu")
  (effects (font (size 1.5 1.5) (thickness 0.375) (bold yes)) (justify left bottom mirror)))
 (segment (start 160.66 66.41) (end 162.04 65.03) (width 0.762) (layer "B.Cu") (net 1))
 (segment (start 165.82 82.1) (end 165.82 83.4447) (width 0.762) (layer "B.Cu") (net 1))
 (segment (start 179.48 83.055) (end 179.48 86.35) (width 0.762) (layer "B.Cu") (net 1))
 (segment (start 162.04 65.03) (end 171.24 65.03) (width 0.762) (layer "B.Cu") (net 1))
 (segment (start 179.48 86.35) (end 179.48 87.962) (width 0.762) (layer "B.Cu") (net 1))
 (segment (start 176.832 90.61) (end 170.6127 90.61) (width 0.762) (layer "B.Cu") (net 1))
 (segment (start 165.82 83.4447) (end 164.9 84.3647) (width 0.762) (layer "B.Cu") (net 1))
 (segment (start 160.66 69.08) (end 160.66 66.41) (width 0.762) (layer "B.Cu") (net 1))
 (segment (start 165.82 71.94) (end 163.52 71.94) (width 0.762) (layer "B.Cu") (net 1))
 (segment (start 166.3327 86.33) (end 164.9 86.33) (width 0.762) (layer "B.Cu") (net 1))
 (segment (start 170.6127 90.61) (end 166.3327 86.33) (width 0.762) (layer "B.Cu") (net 1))
 (segment (start 178.79 82.365) (end 179.48 83.055) (width 0.762) (layer "B.Cu") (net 1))
 (segment (start 171.24 65.03) (end 178.79 72.58) (width 0.762) (layer "B.Cu") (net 1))
 (segment (start 179.48 87.962) (end 176.832 90.61) (width 0.762) (layer "B.Cu") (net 1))
 (segment (start 178.79 80.25) (end 178.79 82.365) (width 0.762) (layer "B.Cu") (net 1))
 (segment (start 163.52 71.94) (end 160.66 69.08) (width 0.762) (layer "B.Cu") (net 1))
 (segment (start 164.9 84.3647) (end 164.9 86.33) (width 0.762) (layer "B.Cu") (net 1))
 (segment (start 178.79 72.58) (end 178.79 80.25) (width 0.762) (layer "B.Cu") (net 1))
 (segment (start 157.28 78.68) (end 157.28 86.33) (width 0.762) (layer "B.Cu") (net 7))
 (segment (start 165.82 74.48) (end 161.48 74.48) (width 0.762) (layer "B.Cu") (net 7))
 (segment (start 161.48 74.48) (end 157.28 78.68) (width 0.762) (layer "B.Cu") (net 7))
 (segment (start 170.5037 80.25) (end 171.86 81.6063) (width 0.762) (layer "B.Cu") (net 4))
 (segment (start 169.75 70.4) (end 169.75 76.5581) (width 0.762) (layer "B.Cu") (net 4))
 (segment (start 171.86 81.6063) (end 171.86 86.35) (width 0.762) (layer "B.Cu") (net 4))
 (segment (start 170.5037 80.25) (end 169.8373 80.25) (width 0.762) (layer "B.Cu") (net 4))
 (segment (start 167.1791 79.129) (end 168.7163 79.129) (width 0.762) (layer "B.Cu") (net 4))
 (segment (start 167.1791 79.129) (end 166.251 79.129) (width 0.762) (layer "B.Cu") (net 4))
 (segment (start 166.251 79.129) (end 165.82 79.56) (width 0.762) (layer "B.Cu") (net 4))
 (segment (start 162.36 81.59) (end 162.36 86.33) (width 0.762) (layer "B.Cu") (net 4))
 (segment (start 165.82 69.4) (end 168.75 69.4) (width 0.762) (layer "B.Cu") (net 4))
 (segment (start 168.75 69.4) (end 169.75 70.4) (width 0.762) (layer "B.Cu") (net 4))
 (segment (start 168.7163 79.129) (end 169.8373 80.25) (width 0.762) (layer "B.Cu") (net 4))
 (segment (start 169.75 76.5581) (end 167.1791 79.129) (width 0.762) (layer "B.Cu") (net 4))
 (segment (start 165.82 79.56) (end 164.39 79.56) (width 0.762) (layer "B.Cu") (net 4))
 (segment (start 171.17 80.25) (end 170.5037 80.25) (width 0.762) (layer "B.Cu") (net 4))
 (segment (start 164.39 79.56) (end 162.36 81.59) (width 0.762) (layer "B.Cu") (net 4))
 (segment (start 162.71 77.02) (end 159.82 79.91) (width 0.762) (layer "B.Cu") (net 6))
 (segment (start 165.82 77.02) (end 162.71 77.02) (width 0.762) (layer "B.Cu") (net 6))
 (segment (start 159.82 79.91) (end 159.82 86.33) (width 0.762) (layer "B.Cu") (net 6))
 (segment (start 173.71 80.25) (end 173.71 81.6873) (width 0.762) (layer "B.Cu") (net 2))
 (segment (start 173.71 81.6873) (end 176.94 84.9173) (width 0.762) (layer "B.Cu") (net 2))
 (segment (start 176.94 86.35) (end 176.94 84.9173) (width 0.762) (layer "B.Cu") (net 2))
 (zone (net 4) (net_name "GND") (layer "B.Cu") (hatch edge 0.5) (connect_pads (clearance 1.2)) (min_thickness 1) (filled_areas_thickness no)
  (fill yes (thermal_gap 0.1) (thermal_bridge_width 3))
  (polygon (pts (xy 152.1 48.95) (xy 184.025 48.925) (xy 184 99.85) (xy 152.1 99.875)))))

